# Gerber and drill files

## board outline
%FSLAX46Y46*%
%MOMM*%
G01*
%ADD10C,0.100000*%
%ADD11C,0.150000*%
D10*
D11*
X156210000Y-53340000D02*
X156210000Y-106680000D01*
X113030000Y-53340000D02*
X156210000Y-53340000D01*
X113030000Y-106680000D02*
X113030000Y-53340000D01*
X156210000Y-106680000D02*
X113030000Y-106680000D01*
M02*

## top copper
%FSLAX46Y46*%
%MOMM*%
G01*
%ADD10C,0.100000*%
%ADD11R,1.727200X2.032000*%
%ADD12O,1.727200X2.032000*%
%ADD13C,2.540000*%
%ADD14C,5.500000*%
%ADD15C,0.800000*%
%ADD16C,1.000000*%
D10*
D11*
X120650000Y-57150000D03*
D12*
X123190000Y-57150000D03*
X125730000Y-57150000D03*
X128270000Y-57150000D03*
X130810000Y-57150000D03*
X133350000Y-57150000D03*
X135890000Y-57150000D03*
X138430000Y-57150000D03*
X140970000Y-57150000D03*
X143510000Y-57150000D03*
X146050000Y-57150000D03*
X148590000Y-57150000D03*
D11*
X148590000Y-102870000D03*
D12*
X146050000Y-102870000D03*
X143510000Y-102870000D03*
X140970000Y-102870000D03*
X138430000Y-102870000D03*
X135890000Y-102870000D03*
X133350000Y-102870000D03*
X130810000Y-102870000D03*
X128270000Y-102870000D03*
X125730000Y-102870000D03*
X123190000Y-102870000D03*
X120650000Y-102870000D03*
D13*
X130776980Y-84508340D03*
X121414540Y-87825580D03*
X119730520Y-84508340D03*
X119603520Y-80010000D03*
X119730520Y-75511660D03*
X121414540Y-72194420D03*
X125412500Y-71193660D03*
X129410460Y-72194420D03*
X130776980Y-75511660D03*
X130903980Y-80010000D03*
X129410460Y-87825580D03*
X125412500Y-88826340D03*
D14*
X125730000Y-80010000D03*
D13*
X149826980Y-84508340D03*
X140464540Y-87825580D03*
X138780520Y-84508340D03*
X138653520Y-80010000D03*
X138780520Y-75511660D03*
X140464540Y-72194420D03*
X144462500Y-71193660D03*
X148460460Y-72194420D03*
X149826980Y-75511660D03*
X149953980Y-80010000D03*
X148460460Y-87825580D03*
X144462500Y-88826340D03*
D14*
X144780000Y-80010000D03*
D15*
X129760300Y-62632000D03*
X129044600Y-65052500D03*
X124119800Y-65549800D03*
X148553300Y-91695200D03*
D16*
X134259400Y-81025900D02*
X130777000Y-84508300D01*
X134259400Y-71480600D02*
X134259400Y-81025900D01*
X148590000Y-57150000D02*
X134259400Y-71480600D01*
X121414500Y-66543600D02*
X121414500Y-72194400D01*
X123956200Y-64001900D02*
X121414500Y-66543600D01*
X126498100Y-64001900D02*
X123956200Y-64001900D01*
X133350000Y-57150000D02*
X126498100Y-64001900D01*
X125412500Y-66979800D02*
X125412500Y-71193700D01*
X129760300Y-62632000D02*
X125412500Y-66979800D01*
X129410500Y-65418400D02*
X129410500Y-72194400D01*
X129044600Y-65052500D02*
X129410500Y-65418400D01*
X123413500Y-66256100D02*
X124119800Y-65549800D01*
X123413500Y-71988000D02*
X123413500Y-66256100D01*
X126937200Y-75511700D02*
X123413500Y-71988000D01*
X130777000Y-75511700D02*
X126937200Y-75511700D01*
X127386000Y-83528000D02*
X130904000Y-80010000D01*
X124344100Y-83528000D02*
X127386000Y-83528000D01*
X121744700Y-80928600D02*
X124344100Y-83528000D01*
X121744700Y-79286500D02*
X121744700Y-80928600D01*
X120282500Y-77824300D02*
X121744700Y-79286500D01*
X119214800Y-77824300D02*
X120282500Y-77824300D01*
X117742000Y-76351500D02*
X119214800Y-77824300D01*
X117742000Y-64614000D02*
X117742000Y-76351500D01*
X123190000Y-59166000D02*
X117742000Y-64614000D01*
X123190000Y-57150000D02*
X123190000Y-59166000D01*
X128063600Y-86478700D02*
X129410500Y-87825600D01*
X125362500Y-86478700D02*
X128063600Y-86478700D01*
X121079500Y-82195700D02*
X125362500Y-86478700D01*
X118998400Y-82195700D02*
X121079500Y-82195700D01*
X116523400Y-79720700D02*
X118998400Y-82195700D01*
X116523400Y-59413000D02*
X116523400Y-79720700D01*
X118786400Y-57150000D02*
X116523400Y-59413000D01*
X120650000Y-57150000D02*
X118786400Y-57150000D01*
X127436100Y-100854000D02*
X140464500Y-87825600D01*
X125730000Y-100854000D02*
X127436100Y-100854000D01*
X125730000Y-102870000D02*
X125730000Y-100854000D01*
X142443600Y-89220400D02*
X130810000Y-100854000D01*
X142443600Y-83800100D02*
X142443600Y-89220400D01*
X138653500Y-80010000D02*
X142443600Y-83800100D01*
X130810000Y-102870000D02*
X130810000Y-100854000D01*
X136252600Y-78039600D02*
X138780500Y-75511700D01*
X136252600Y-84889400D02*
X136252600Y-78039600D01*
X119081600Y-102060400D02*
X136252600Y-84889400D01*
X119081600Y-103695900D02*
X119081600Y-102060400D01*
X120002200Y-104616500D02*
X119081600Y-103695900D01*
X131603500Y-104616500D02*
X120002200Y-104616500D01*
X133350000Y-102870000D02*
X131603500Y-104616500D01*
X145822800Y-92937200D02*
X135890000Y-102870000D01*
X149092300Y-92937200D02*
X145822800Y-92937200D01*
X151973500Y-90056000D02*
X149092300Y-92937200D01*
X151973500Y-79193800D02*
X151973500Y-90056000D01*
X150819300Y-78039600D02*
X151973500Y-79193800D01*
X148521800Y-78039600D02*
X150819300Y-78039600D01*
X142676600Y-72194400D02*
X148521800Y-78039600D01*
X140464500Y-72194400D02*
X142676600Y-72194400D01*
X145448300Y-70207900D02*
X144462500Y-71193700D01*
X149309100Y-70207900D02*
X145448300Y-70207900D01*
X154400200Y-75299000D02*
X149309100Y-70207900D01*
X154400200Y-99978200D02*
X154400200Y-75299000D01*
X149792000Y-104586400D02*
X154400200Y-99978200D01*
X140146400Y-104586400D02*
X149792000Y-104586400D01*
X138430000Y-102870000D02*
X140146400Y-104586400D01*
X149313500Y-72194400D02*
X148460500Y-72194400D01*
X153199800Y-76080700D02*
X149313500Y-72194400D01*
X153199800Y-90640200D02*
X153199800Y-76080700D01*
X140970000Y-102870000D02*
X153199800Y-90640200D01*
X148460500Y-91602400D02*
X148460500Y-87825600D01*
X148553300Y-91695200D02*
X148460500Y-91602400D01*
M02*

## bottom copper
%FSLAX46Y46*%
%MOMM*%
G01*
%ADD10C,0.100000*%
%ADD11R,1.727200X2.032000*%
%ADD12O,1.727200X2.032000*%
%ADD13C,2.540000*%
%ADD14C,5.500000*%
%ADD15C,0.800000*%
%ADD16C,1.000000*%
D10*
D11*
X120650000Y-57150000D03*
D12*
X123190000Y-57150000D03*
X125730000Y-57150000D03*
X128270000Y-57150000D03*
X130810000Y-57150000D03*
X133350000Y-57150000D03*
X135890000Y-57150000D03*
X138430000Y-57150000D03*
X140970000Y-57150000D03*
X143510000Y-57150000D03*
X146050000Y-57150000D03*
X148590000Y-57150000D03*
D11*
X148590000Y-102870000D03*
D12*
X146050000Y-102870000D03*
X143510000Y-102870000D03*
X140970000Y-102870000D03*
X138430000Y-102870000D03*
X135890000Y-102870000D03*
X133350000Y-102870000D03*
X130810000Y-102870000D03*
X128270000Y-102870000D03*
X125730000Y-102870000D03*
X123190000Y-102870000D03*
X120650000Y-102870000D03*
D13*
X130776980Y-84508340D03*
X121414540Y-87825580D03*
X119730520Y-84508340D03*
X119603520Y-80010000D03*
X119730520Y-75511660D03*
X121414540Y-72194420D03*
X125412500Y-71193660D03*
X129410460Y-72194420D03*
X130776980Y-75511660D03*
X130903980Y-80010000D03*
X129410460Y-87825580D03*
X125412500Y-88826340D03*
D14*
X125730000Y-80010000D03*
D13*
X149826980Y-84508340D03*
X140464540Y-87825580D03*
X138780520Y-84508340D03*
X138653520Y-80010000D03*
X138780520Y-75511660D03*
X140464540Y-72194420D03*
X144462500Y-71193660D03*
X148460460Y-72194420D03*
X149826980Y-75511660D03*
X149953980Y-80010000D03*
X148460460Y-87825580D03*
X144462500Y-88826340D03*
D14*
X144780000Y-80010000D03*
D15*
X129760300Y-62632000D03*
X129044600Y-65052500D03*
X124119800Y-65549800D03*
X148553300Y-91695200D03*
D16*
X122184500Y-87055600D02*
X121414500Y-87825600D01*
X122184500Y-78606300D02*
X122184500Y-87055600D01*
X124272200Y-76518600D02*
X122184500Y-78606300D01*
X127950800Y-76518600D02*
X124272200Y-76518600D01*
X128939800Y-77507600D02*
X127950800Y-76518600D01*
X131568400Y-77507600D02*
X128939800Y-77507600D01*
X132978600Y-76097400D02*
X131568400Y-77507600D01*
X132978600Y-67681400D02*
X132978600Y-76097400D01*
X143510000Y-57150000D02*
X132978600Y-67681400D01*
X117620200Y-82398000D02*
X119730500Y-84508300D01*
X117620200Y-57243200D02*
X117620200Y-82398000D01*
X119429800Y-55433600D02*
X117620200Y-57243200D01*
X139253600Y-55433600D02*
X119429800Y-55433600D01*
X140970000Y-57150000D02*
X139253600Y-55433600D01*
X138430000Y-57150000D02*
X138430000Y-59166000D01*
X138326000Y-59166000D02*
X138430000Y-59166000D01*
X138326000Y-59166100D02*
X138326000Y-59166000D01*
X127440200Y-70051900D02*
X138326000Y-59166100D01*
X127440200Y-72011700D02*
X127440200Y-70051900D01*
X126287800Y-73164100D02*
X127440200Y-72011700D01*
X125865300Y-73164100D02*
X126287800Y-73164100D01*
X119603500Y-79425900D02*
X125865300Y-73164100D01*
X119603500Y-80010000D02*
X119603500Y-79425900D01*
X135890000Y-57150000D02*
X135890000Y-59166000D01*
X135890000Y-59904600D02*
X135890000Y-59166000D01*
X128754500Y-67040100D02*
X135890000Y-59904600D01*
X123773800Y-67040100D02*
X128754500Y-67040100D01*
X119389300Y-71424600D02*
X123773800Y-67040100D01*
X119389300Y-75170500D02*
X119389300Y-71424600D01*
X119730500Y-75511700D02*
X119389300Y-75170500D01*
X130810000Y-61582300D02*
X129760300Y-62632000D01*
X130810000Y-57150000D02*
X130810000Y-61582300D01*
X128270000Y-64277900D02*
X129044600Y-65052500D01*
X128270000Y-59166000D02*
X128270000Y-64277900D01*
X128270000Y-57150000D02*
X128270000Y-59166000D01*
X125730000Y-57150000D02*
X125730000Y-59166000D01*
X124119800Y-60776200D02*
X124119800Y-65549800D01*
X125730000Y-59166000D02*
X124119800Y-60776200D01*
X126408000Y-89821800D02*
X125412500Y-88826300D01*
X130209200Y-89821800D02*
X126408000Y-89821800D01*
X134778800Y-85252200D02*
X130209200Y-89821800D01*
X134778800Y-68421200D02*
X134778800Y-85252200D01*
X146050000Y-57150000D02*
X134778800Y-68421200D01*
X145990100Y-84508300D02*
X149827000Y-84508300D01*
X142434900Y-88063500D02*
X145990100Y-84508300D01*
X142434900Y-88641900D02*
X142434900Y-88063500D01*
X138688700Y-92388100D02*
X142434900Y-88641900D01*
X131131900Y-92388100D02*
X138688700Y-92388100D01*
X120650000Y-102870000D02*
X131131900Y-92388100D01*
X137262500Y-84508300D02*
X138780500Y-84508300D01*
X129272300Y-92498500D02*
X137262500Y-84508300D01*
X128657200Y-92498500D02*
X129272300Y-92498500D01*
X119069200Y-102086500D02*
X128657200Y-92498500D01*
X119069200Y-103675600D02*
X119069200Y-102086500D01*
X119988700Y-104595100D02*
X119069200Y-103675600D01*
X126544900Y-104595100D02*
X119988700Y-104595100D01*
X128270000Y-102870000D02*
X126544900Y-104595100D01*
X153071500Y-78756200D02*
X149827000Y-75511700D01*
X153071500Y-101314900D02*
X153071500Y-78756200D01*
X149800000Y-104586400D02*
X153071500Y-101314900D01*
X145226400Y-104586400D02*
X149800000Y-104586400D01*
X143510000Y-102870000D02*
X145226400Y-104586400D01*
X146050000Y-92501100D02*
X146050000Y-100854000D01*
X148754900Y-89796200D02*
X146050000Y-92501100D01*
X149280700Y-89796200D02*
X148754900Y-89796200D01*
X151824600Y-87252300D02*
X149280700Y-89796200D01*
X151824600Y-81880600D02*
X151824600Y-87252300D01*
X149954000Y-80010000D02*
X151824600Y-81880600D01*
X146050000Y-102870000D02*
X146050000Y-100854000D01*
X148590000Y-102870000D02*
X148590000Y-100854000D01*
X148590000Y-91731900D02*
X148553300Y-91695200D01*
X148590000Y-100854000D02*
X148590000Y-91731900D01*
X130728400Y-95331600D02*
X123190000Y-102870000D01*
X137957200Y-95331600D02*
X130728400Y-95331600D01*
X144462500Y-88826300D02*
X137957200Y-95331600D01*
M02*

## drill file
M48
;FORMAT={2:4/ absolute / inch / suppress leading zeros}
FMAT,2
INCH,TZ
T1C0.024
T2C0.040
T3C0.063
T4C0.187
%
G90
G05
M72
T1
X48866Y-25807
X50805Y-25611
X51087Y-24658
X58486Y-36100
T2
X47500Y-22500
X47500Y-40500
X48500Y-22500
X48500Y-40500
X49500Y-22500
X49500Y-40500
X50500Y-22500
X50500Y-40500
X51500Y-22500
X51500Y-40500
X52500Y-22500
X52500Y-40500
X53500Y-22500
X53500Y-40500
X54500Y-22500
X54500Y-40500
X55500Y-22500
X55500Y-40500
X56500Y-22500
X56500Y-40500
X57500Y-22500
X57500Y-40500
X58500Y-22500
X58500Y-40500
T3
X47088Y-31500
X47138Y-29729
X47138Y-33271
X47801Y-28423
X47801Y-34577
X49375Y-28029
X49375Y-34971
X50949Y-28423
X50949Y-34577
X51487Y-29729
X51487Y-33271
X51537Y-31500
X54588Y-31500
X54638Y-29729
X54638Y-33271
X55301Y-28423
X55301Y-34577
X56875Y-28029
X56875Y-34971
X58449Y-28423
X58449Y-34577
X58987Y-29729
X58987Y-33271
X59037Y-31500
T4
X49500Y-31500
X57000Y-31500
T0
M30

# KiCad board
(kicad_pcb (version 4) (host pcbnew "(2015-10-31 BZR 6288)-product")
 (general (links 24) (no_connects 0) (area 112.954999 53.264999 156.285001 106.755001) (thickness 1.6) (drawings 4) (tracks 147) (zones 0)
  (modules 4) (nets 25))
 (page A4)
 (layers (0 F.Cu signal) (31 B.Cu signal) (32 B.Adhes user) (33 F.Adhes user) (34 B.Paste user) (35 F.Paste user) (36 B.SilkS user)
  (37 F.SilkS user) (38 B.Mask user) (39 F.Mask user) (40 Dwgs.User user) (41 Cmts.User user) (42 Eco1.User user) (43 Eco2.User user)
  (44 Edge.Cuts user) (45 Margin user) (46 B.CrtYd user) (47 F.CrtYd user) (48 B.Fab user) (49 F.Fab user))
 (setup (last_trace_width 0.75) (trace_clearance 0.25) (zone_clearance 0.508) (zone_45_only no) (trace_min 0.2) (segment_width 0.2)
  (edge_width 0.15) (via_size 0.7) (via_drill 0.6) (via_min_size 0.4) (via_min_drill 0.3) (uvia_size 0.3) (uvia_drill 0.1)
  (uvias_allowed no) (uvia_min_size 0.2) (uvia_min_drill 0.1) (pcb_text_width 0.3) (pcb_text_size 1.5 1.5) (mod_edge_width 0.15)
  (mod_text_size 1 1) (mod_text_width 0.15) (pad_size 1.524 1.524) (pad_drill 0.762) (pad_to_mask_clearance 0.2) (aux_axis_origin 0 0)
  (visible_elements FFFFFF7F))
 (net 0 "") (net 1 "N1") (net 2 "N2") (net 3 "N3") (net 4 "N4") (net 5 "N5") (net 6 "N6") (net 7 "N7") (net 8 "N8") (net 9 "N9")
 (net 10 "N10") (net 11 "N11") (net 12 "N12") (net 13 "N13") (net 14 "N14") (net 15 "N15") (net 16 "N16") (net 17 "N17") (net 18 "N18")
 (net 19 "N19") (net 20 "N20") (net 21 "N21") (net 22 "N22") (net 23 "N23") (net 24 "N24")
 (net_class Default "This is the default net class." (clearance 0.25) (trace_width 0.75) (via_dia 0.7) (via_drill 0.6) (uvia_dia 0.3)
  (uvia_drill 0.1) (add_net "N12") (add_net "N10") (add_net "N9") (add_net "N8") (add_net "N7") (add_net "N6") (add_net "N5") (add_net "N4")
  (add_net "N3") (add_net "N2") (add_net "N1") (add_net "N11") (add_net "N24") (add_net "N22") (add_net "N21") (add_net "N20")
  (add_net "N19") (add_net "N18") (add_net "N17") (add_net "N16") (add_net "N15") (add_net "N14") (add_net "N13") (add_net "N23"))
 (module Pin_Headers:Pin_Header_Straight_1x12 (layer F.Cu) (at 120.65 57.15 90)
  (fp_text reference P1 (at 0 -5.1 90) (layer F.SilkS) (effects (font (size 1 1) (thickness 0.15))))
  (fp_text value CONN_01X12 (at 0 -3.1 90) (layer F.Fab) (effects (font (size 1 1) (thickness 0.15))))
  (pad 1 thru_hole rect (at 0 0 90) (size 2.032 1.7272) (drill 1.016) (layers *.Cu *.Mask F.SilkS) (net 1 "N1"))
  (pad 2 thru_hole oval (at 0 2.54 90) (size 2.032 1.7272) (drill 1.016) (layers *.Cu *.Mask F.SilkS) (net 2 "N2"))
  (pad 3 thru_hole oval (at 0 5.08 90) (size 2.032 1.7272) (drill 1.016) (layers *.Cu *.Mask F.SilkS) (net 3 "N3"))
  (pad 4 thru_hole oval (at 0 7.62 90) (size 2.032 1.7272) (drill 1.016) (layers *.Cu *.Mask F.SilkS) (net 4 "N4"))
  (pad 5 thru_hole oval (at 0 10.16 90) (size 2.032 1.7272) (drill 1.016) (layers *.Cu *.Mask F.SilkS) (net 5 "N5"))
  (pad 6 thru_hole oval (at 0 12.7 90) (size 2.032 1.7272) (drill 1.016) (layers *.Cu *.Mask F.SilkS) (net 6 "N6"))
  (pad 7 thru_hole oval (at 0 15.24 90) (size 2.032 1.7272) (drill 1.016) (layers *.Cu *.Mask F.SilkS) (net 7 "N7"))
  (pad 8 thru_hole oval (at 0 17.78 90) (size 2.032 1.7272) (drill 1.016) (layers *.Cu *.Mask F.SilkS) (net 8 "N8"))
  (pad 9 thru_hole oval (at 0 20.32 90) (size 2.032 1.7272) (drill 1.016) (layers *.Cu *.Mask F.SilkS) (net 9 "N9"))
  (pad 10 thru_hole oval (at 0 22.86 90) (size 2.032 1.7272) (drill 1.016) (layers *.Cu *.Mask F.SilkS) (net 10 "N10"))
  (pad 11 thru_hole oval (at 0 25.4 90) (size 2.032 1.7272) (drill 1.016) (layers *.Cu *.Mask F.SilkS) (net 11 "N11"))
  (pad 12 thru_hole oval (at 0 27.94 90) (size 2.032 1.7272) (drill 1.016) (layers *.Cu *.Mask F.SilkS) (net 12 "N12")))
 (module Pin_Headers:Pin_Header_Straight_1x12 (layer F.Cu) (at 148.59 102.87 270)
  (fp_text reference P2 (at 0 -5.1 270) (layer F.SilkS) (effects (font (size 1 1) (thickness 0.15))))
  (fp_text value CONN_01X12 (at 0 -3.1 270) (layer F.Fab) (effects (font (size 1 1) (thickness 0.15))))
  (pad 1 thru_hole rect (at 0 0 270) (size 2.032 1.7272) (drill 1.016) (layers *.Cu *.Mask F.SilkS) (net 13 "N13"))
  (pad 2 thru_hole oval (at 0 2.54 270) (size 2.032 1.7272) (drill 1.016) (layers *.Cu *.Mask F.SilkS) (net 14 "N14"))
  (pad 3 thru_hole oval (at 0 5.08 270) (size 2.032 1.7272) (drill 1.016) (layers *.Cu *.Mask F.SilkS) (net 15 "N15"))
  (pad 4 thru_hole oval (at 0 7.62 270) (size 2.032 1.7272) (drill 1.016) (layers *.Cu *.Mask F.SilkS) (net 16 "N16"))
  (pad 5 thru_hole oval (at 0 10.16 270) (size 2.032 1.7272) (drill 1.016) (layers *.Cu *.Mask F.SilkS) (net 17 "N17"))
  (pad 6 thru_hole oval (at 0 12.7 270) (size 2.032 1.7272) (drill 1.016) (layers *.Cu *.Mask F.SilkS) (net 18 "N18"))
  (pad 7 thru_hole oval (at 0 15.24 270) (size 2.032 1.7272) (drill 1.016) (layers *.Cu *.Mask F.SilkS) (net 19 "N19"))
  (pad 8 thru_hole oval (at 0 17.78 270) (size 2.032 1.7272) (drill 1.016) (layers *.Cu *.Mask F.SilkS) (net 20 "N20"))
  (pad 9 thru_hole oval (at 0 20.32 270) (size 2.032 1.7272) (drill 1.016) (layers *.Cu *.Mask F.SilkS) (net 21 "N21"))
  (pad 10 thru_hole oval (at 0 22.86 270) (size 2.032 1.7272) (drill 1.016) (layers *.Cu *.Mask F.SilkS) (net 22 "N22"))
  (pad 11 thru_hole oval (at 0 25.4 270) (size 2.032 1.7272) (drill 1.016) (layers *.Cu *.Mask F.SilkS) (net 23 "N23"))
  (pad 12 thru_hole oval (at 0 27.94 270) (size 2.032 1.7272) (drill 1.016) (layers *.Cu *.Mask F.SilkS) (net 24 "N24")))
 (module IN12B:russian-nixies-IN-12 (layer F.Cu) (at 125.73 80.01)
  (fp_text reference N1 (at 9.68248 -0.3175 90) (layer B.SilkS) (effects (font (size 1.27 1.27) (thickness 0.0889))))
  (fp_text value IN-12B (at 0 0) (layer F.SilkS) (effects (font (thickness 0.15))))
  (pad 0 thru_hole circle (at 5.04698 4.49834) (size 2.54 2.54) (drill 1.6) (layers *.Cu *.Mask F.SilkS) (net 12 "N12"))
  (pad 1 thru_hole circle (at -4.31546 7.81558) (size 2.54 2.54) (drill 1.6) (layers *.Cu *.Mask F.SilkS) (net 10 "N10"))
  (pad 2 thru_hole circle (at -5.99948 4.49834) (size 2.54 2.54) (drill 1.6) (layers *.Cu *.Mask F.SilkS) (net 9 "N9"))
  (pad 3 thru_hole circle (at -6.12648 0) (size 2.54 2.54) (drill 1.6) (layers *.Cu *.Mask F.SilkS) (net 8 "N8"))
  (pad 4 thru_hole circle (at -5.99948 -4.49834) (size 2.54 2.54) (drill 1.6) (layers *.Cu *.Mask F.SilkS) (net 7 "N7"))
  (pad 5 thru_hole circle (at -4.31546 -7.81558) (size 2.54 2.54) (drill 1.6) (layers *.Cu *.Mask F.SilkS) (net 6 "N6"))
  (pad 6 thru_hole circle (at -0.3175 -8.81634) (size 2.54 2.54) (drill 1.6) (layers *.Cu *.Mask F.SilkS) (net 5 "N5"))
  (pad 7 thru_hole circle (at 3.68046 -7.81558) (size 2.54 2.54) (drill 1.6) (layers *.Cu *.Mask F.SilkS) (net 4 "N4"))
  (pad 8 thru_hole circle (at 5.04698 -4.49834) (size 2.54 2.54) (drill 1.6) (layers *.Cu *.Mask F.SilkS) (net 3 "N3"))
  (pad 9 thru_hole circle (at 5.17398 0) (size 2.54 2.54) (drill 1.6) (layers *.Cu *.Mask F.SilkS) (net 2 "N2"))
  (pad A thru_hole circle (at 3.68046 7.81558) (size 2.54 2.54) (drill 1.6) (layers *.Cu *.Mask F.SilkS) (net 1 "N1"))
  (pad LHDP thru_hole circle (at -0.3175 8.81634) (size 2.54 2.54) (drill 1.6) (layers *.Cu *.Mask F.SilkS) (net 11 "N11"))
  (pad "" thru_hole circle (at 0 0) (size 5.5 5.5) (drill 4.75) (layers *.Cu)))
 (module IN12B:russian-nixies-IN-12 (layer F.Cu) (at 144.78 80.01)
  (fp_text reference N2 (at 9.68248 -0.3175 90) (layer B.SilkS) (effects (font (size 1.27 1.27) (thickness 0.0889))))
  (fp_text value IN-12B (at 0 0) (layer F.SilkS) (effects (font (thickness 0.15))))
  (pad 0 thru_hole circle (at 5.04698 4.49834) (size 2.54 2.54) (drill 1.6) (layers *.Cu *.Mask F.SilkS) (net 24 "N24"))
  (pad 1 thru_hole circle (at -4.31546 7.81558) (size 2.54 2.54) (drill 1.6) (layers *.Cu *.Mask F.SilkS) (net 22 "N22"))
  (pad 2 thru_hole circle (at -5.99948 4.49834) (size 2.54 2.54) (drill 1.6) (layers *.Cu *.Mask F.SilkS) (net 21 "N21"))
  (pad 3 thru_hole circle (at -6.12648 0) (size 2.54 2.54) (drill 1.6) (layers *.Cu *.Mask F.SilkS) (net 20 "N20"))
  (pad 4 thru_hole circle (at -5.99948 -4.49834) (size 2.54 2.54) (drill 1.6) (layers *.Cu *.Mask F.SilkS) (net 19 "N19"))
  (pad 5 thru_hole circle (at -4.31546 -7.81558) (size 2.54 2.54) (drill 1.6) (layers *.Cu *.Mask F.SilkS) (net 18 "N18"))
  (pad 6 thru_hole circle (at -0.3175 -8.81634) (size 2.54 2.54) (drill 1.6) (layers *.Cu *.Mask F.SilkS) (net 17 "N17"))
  (pad 7 thru_hole circle (at 3.68046 -7.81558) (size 2.54 2.54) (drill 1.6) (layers *.Cu *.Mask F.SilkS) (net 16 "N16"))
  (pad 8 thru_hole circle (at 5.04698 -4.49834) (size 2.54 2.54) (drill 1.6) (layers *.Cu *.Mask F.SilkS) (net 15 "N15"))
  (pad 9 thru_hole circle (at 5.17398 0) (size 2.54 2.54) (drill 1.6) (layers *.Cu *.Mask F.SilkS) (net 14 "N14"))
  (pad A thru_hole circle (at 3.68046 7.81558) (size 2.54 2.54) (drill 1.6) (layers *.Cu *.Mask F.SilkS) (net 13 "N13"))
  (pad LHDP thru_hole circle (at -0.3175 8.81634) (size 2.54 2.54) (drill 1.6) (layers *.Cu *.Mask F.SilkS) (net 23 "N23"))
  (pad "" thru_hole circle (at 0 0) (size 5.5 5.5) (drill 4.75) (layers *.Cu)))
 (gr_line (start 156.21 53.34) (end 156.21 106.68) (angle 90) (layer Edge.Cuts) (width 0.15))
 (gr_line (start 113.03 53.34) (end 156.21 53.34) (angle 90) (layer Edge.Cuts) (width 0.15))
 (gr_line (start 113.03 106.68) (end 113.03 53.34) (angle 90) (layer Edge.Cuts) (width 0.15))
 (gr_line (start 156.21 106.68) (end 113.03 106.68) (angle 90) (layer Edge.Cuts) (width 0.15))
 (segment (start 134.2594 81.0259) (end 130.777 84.5083) (width 1) (layer F.Cu) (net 12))
 (segment (start 134.2594 71.4806) (end 134.2594 81.0259) (width 1) (layer F.Cu) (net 12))
 (segment (start 148.59 57.15) (end 134.2594 71.4806) (width 1) (layer F.Cu) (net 12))
 (segment (start 122.1845 87.0556) (end 121.4145 87.8256) (width 1) (layer B.Cu) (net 10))
 (segment (start 122.1845 78.6063) (end 122.1845 87.0556) (width 1) (layer B.Cu) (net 10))
 (segment (start 124.2722 76.5186) (end 122.1845 78.6063) (width 1) (layer B.Cu) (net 10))
 (segment (start 127.9508 76.5186) (end 124.2722 76.5186) (width 1) (layer B.Cu) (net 10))
 (segment (start 128.9398 77.5076) (end 127.9508 76.5186) (width 1) (layer B.Cu) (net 10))
 (segment (start 131.5684 77.5076) (end 128.9398 77.5076) (width 1) (layer B.Cu) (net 10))
 (segment (start 132.9786 76.0974) (end 131.5684 77.5076) (width 1) (layer B.Cu) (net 10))
 (segment (start 132.9786 67.6814) (end 132.9786 76.0974) (width 1) (layer B.Cu) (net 10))
 (segment (start 143.51 57.15) (end 132.9786 67.6814) (width 1) (layer B.Cu) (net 10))
 (segment (start 117.6202 82.398) (end 119.7305 84.5083) (width 1) (layer B.Cu) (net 9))
 (segment (start 117.6202 57.2432) (end 117.6202 82.398) (width 1) (layer B.Cu) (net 9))
 (segment (start 119.4298 55.4336) (end 117.6202 57.2432) (width 1) (layer B.Cu) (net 9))
 (segment (start 139.2536 55.4336) (end 119.4298 55.4336) (width 1) (layer B.Cu) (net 9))
 (segment (start 140.97 57.15) (end 139.2536 55.4336) (width 1) (layer B.Cu) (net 9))
 (segment (start 138.43 57.15) (end 138.43 59.166) (width 1) (layer B.Cu) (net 8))
 (segment (start 138.326 59.166) (end 138.43 59.166) (width 1) (layer B.Cu) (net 8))
 (segment (start 138.326 59.1661) (end 138.326 59.166) (width 1) (layer B.Cu) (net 8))
 (segment (start 127.4402 70.0519) (end 138.326 59.1661) (width 1) (layer B.Cu) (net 8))
 (segment (start 127.4402 72.0117) (end 127.4402 70.0519) (width 1) (layer B.Cu) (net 8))
 (segment (start 126.2878 73.1641) (end 127.4402 72.0117) (width 1) (layer B.Cu) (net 8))
 (segment (start 125.8653 73.1641) (end 126.2878 73.1641) (width 1) (layer B.Cu) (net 8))
 (segment (start 119.6035 79.4259) (end 125.8653 73.1641) (width 1) (layer B.Cu) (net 8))
 (segment (start 119.6035 80.01) (end 119.6035 79.4259) (width 1) (layer B.Cu) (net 8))
 (segment (start 135.89 57.15) (end 135.89 59.166) (width 1) (layer B.Cu) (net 7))
 (segment (start 135.89 59.9046) (end 135.89 59.166) (width 1) (layer B.Cu) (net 7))
 (segment (start 128.7545 67.0401) (end 135.89 59.9046) (width 1) (layer B.Cu) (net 7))
 (segment (start 123.7738 67.0401) (end 128.7545 67.0401) (width 1) (layer B.Cu) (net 7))
 (segment (start 119.3893 71.4246) (end 123.7738 67.0401) (width 1) (layer B.Cu) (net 7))
 (segment (start 119.3893 75.1705) (end 119.3893 71.4246) (width 1) (layer B.Cu) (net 7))
 (segment (start 119.7305 75.5117) (end 119.3893 75.1705) (width 1) (layer B.Cu) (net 7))
 (segment (start 121.4145 66.5436) (end 121.4145 72.1944) (width 1) (layer F.Cu) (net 6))
 (segment (start 123.9562 64.0019) (end 121.4145 66.5436) (width 1) (layer F.Cu) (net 6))
 (segment (start 126.4981 64.0019) (end 123.9562 64.0019) (width 1) (layer F.Cu) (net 6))
 (segment (start 133.35 57.15) (end 126.4981 64.0019) (width 1) (layer F.Cu) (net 6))
 (via (at 129.7603 62.632) (size 0.8) (layers F.Cu B.Cu) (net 5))
 (segment (start 130.81 61.5823) (end 129.7603 62.632) (width 1) (layer B.Cu) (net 5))
 (segment (start 130.81 57.15) (end 130.81 61.5823) (width 1) (layer B.Cu) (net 5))
 (segment (start 125.4125 66.9798) (end 125.4125 71.1937) (width 1) (layer F.Cu) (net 5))
 (segment (start 129.7603 62.632) (end 125.4125 66.9798) (width 1) (layer F.Cu) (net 5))
 (via (at 129.0446 65.0525) (size 0.8) (layers F.Cu B.Cu) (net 4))
 (segment (start 128.27 64.2779) (end 129.0446 65.0525) (width 1) (layer B.Cu) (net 4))
 (segment (start 128.27 59.166) (end 128.27 64.2779) (width 1) (layer B.Cu) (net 4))
 (segment (start 129.4105 65.4184) (end 129.4105 72.1944) (width 1) (layer F.Cu) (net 4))
 (segment (start 129.0446 65.0525) (end 129.4105 65.4184) (width 1) (layer F.Cu) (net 4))
 (segment (start 128.27 57.15) (end 128.27 59.166) (width 1) (layer B.Cu) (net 4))
 (via (at 124.1198 65.5498) (size 0.8) (layers F.Cu B.Cu) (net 3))
 (segment (start 125.73 57.15) (end 125.73 59.166) (width 1) (layer B.Cu) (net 3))
 (segment (start 124.1198 60.7762) (end 124.1198 65.5498) (width 1) (layer B.Cu) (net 3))
 (segment (start 125.73 59.166) (end 124.1198 60.7762) (width 1) (layer B.Cu) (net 3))
 (segment (start 123.4135 66.2561) (end 124.1198 65.5498) (width 1) (layer F.Cu) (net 3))
 (segment (start 123.4135 71.988) (end 123.4135 66.2561) (width 1) (layer F.Cu) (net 3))
 (segment (start 126.9372 75.5117) (end 123.4135 71.988) (width 1) (layer F.Cu) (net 3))
 (segment (start 130.777 75.5117) (end 126.9372 75.5117) (width 1) (layer F.Cu) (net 3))
 (segment (start 127.386 83.528) (end 130.904 80.01) (width 1) (layer F.Cu) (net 2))
 (segment (start 124.3441 83.528) (end 127.386 83.528) (width 1) (layer F.Cu) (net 2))
 (segment (start 121.7447 80.9286) (end 124.3441 83.528) (width 1) (layer F.Cu) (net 2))
 (segment (start 121.7447 79.2865) (end 121.7447 80.9286) (width 1) (layer F.Cu) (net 2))
 (segment (start 120.2825 77.8243) (end 121.7447 79.2865) (width 1) (layer F.Cu) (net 2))
 (segment (start 119.2148 77.8243) (end 120.2825 77.8243) (width 1) (layer F.Cu) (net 2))
 (segment (start 117.742 76.3515) (end 119.2148 77.8243) (width 1) (layer F.Cu) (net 2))
 (segment (start 117.742 64.614) (end 117.742 76.3515) (width 1) (layer F.Cu) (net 2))
 (segment (start 123.19 59.166) (end 117.742 64.614) (width 1) (layer F.Cu) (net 2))
 (segment (start 123.19 57.15) (end 123.19 59.166) (width 1) (layer F.Cu) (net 2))
 (segment (start 128.0636 86.4787) (end 129.4105 87.8256) (width 1) (layer F.Cu) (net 1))
 (segment (start 125.3625 86.4787) (end 128.0636 86.4787) (width 1) (layer F.Cu) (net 1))
 (segment (start 121.0795 82.1957) (end 125.3625 86.4787) (width 1) (layer F.Cu) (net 1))
 (segment (start 118.9984 82.1957) (end 121.0795 82.1957) (width 1) (layer F.Cu) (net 1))
 (segment (start 116.5234 79.7207) (end 118.9984 82.1957) (width 1) (layer F.Cu) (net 1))
 (segment (start 116.5234 59.413) (end 116.5234 79.7207) (width 1) (layer F.Cu) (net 1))
 (segment (start 118.7864 57.15) (end 116.5234 59.413) (width 1) (layer F.Cu) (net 1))
 (segment (start 120.65 57.15) (end 118.7864 57.15) (width 1) (layer F.Cu) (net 1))
 (segment (start 126.408 89.8218) (end 125.4125 88.8263) (width 1) (layer B.Cu) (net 11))
 (segment (start 130.2092 89.8218) (end 126.408 89.8218) (width 1) (layer B.Cu) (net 11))
 (segment (start 134.7788 85.2522) (end 130.2092 89.8218) (width 1) (layer B.Cu) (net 11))
 (segment (start 134.7788 68.4212) (end 134.7788 85.2522) (width 1) (layer B.Cu) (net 11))
 (segment (start 146.05 57.15) (end 134.7788 68.4212) (width 1) (layer B.Cu) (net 11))
 (segment (start 145.9901 84.5083) (end 149.827 84.5083) (width 1) (layer B.Cu) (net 24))
 (segment (start 142.4349 88.0635) (end 145.9901 84.5083) (width 1) (layer B.Cu) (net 24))
 (segment (start 142.4349 88.6419) (end 142.4349 88.0635) (width 1) (layer B.Cu) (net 24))
 (segment (start 138.6887 92.3881) (end 142.4349 88.6419) (width 1) (layer B.Cu) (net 24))
 (segment (start 131.1319 92.3881) (end 138.6887 92.3881) (width 1) (layer B.Cu) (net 24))
 (segment (start 120.65 102.87) (end 131.1319 92.3881) (width 1) (layer B.Cu) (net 24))
 (segment (start 127.4361 100.854) (end 140.4645 87.8256) (width 1) (layer F.Cu) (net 22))
 (segment (start 125.73 100.854) (end 127.4361 100.854) (width 1) (layer F.Cu) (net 22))
 (segment (start 125.73 102.87) (end 125.73 100.854) (width 1) (layer F.Cu) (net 22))
 (segment (start 137.2625 84.5083) (end 138.7805 84.5083) (width 1) (layer B.Cu) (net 21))
 (segment (start 129.2723 92.4985) (end 137.2625 84.5083) (width 1) (layer B.Cu) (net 21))
 (segment (start 128.6572 92.4985) (end 129.2723 92.4985) (width 1) (layer B.Cu) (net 21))
 (segment (start 119.0692 102.0865) (end 128.6572 92.4985) (width 1) (layer B.Cu) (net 21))
 (segment (start 119.0692 103.6756) (end 119.0692 102.0865) (width 1) (layer B.Cu) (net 21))
 (segment (start 119.9887 104.5951) (end 119.0692 103.6756) (width 1) (layer B.Cu) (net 21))
 (segment (start 126.5449 104.5951) (end 119.9887 104.5951) (width 1) (layer B.Cu) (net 21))
 (segment (start 128.27 102.87) (end 126.5449 104.5951) (width 1) (layer B.Cu) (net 21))
 (segment (start 142.4436 89.2204) (end 130.81 100.854) (width 1) (layer F.Cu) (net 20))
 (segment (start 142.4436 83.8001) (end 142.4436 89.2204) (width 1) (layer F.Cu) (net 20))
 (segment (start 138.6535 80.01) (end 142.4436 83.8001) (width 1) (layer F.Cu) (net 20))
 (segment (start 130.81 102.87) (end 130.81 100.854) (width 1) (layer F.Cu) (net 20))
 (segment (start 136.2526 78.0396) (end 138.7805 75.5117) (width 1) (layer F.Cu) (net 19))
 (segment (start 136.2526 84.8894) (end 136.2526 78.0396) (width 1) (layer F.Cu) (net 19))
 (segment (start 119.0816 102.0604) (end 136.2526 84.8894) (width 1) (layer F.Cu) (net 19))
 (segment (start 119.0816 103.6959) (end 119.0816 102.0604) (width 1) (layer F.Cu) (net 19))
 (segment (start 120.0022 104.6165) (end 119.0816 103.6959) (width 1) (layer F.Cu) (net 19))
 (segment (start 131.6035 104.6165) (end 120.0022 104.6165) (width 1) (layer F.Cu) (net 19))
 (segment (start 133.35 102.87) (end 131.6035 104.6165) (width 1) (layer F.Cu) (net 19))
 (segment (start 145.8228 92.9372) (end 135.89 102.87) (width 1) (layer F.Cu) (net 18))
 (segment (start 149.0923 92.9372) (end 145.8228 92.9372) (width 1) (layer F.Cu) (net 18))
 (segment (start 151.9735 90.056) (end 149.0923 92.9372) (width 1) (layer F.Cu) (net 18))
 (segment (start 151.9735 79.1938) (end 151.9735 90.056) (width 1) (layer F.Cu) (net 18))
 (segment (start 150.8193 78.0396) (end 151.9735 79.1938) (width 1) (layer F.Cu) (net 18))
 (segment (start 148.5218 78.0396) (end 150.8193 78.0396) (width 1) (layer F.Cu) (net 18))
 (segment (start 142.6766 72.1944) (end 148.5218 78.0396) (width 1) (layer F.Cu) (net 18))
 (segment (start 140.4645 72.1944) (end 142.6766 72.1944) (width 1) (layer F.Cu) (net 18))
 (segment (start 145.4483 70.2079) (end 144.4625 71.1937) (width 1) (layer F.Cu) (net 17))
 (segment (start 149.3091 70.2079) (end 145.4483 70.2079) (width 1) (layer F.Cu) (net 17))
 (segment (start 154.4002 75.299) (end 149.3091 70.2079) (width 1) (layer F.Cu) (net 17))
 (segment (start 154.4002 99.9782) (end 154.4002 75.299) (width 1) (layer F.Cu) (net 17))
 (segment (start 149.792 104.5864) (end 154.4002 99.9782) (width 1) (layer F.Cu) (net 17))
 (segment (start 140.1464 104.5864) (end 149.792 104.5864) (width 1) (layer F.Cu) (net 17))
 (segment (start 138.43 102.87) (end 140.1464 104.5864) (width 1) (layer F.Cu) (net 17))
 (segment (start 149.3135 72.1944) (end 148.4605 72.1944) (width 1) (layer F.Cu) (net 16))
 (segment (start 153.1998 76.0807) (end 149.3135 72.1944) (width 1) (layer F.Cu) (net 16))
 (segment (start 153.1998 90.6402) (end 153.1998 76.0807) (width 1) (layer F.Cu) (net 16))
 (segment (start 140.97 102.87) (end 153.1998 90.6402) (width 1) (layer F.Cu) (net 16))
 (segment (start 153.0715 78.7562) (end 149.827 75.5117) (width 1) (layer B.Cu) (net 15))
 (segment (start 153.0715 101.3149) (end 153.0715 78.7562) (width 1) (layer B.Cu) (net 15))
 (segment (start 149.8 104.5864) (end 153.0715 101.3149) (width 1) (layer B.Cu) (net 15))
 (segment (start 145.2264 104.5864) (end 149.8 104.5864) (width 1) (layer B.Cu) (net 15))
 (segment (start 143.51 102.87) (end 145.2264 104.5864) (width 1) (layer B.Cu) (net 15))
 (segment (start 146.05 92.5011) (end 146.05 100.854) (width 1) (layer B.Cu) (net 14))
 (segment (start 148.7549 89.7962) (end 146.05 92.5011) (width 1) (layer B.Cu) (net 14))
 (segment (start 149.2807 89.7962) (end 148.7549 89.7962) (width 1) (layer B.Cu) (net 14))
 (segment (start 151.8246 87.2523) (end 149.2807 89.7962) (width 1) (layer B.Cu) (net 14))
 (segment (start 151.8246 81.8806) (end 151.8246 87.2523) (width 1) (layer B.Cu) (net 14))
 (segment (start 149.954 80.01) (end 151.8246 81.8806) (width 1) (layer B.Cu) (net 14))
 (segment (start 146.05 102.87) (end 146.05 100.854) (width 1) (layer B.Cu) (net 14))
 (via (at 148.5533 91.6952) (size 0.8) (layers F.Cu B.Cu) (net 13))
 (segment (start 148.59 102.87) (end 148.59 100.854) (width 1) (layer B.Cu) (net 13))
 (segment (start 148.59 91.7319) (end 148.5533 91.6952) (width 1) (layer B.Cu) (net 13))
 (segment (start 148.59 100.854) (end 148.59 91.7319) (width 1) (layer B.Cu) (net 13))
 (segment (start 148.4605 91.6024) (end 148.4605 87.8256) (width 1) (layer F.Cu) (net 13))
 (segment (start 148.5533 91.6952) (end 148.4605 91.6024) (width 1) (layer F.Cu) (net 13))
 (segment (start 130.7284 95.3316) (end 123.19 102.87) (width 1) (layer B.Cu) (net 23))
 (segment (start 137.9572 95.3316) (end 130.7284 95.3316) (width 1) (layer B.Cu) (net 23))
 (segment (start 144.4625 88.8263) (end 137.9572 95.3316) (width 1) (layer B.Cu) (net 23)))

